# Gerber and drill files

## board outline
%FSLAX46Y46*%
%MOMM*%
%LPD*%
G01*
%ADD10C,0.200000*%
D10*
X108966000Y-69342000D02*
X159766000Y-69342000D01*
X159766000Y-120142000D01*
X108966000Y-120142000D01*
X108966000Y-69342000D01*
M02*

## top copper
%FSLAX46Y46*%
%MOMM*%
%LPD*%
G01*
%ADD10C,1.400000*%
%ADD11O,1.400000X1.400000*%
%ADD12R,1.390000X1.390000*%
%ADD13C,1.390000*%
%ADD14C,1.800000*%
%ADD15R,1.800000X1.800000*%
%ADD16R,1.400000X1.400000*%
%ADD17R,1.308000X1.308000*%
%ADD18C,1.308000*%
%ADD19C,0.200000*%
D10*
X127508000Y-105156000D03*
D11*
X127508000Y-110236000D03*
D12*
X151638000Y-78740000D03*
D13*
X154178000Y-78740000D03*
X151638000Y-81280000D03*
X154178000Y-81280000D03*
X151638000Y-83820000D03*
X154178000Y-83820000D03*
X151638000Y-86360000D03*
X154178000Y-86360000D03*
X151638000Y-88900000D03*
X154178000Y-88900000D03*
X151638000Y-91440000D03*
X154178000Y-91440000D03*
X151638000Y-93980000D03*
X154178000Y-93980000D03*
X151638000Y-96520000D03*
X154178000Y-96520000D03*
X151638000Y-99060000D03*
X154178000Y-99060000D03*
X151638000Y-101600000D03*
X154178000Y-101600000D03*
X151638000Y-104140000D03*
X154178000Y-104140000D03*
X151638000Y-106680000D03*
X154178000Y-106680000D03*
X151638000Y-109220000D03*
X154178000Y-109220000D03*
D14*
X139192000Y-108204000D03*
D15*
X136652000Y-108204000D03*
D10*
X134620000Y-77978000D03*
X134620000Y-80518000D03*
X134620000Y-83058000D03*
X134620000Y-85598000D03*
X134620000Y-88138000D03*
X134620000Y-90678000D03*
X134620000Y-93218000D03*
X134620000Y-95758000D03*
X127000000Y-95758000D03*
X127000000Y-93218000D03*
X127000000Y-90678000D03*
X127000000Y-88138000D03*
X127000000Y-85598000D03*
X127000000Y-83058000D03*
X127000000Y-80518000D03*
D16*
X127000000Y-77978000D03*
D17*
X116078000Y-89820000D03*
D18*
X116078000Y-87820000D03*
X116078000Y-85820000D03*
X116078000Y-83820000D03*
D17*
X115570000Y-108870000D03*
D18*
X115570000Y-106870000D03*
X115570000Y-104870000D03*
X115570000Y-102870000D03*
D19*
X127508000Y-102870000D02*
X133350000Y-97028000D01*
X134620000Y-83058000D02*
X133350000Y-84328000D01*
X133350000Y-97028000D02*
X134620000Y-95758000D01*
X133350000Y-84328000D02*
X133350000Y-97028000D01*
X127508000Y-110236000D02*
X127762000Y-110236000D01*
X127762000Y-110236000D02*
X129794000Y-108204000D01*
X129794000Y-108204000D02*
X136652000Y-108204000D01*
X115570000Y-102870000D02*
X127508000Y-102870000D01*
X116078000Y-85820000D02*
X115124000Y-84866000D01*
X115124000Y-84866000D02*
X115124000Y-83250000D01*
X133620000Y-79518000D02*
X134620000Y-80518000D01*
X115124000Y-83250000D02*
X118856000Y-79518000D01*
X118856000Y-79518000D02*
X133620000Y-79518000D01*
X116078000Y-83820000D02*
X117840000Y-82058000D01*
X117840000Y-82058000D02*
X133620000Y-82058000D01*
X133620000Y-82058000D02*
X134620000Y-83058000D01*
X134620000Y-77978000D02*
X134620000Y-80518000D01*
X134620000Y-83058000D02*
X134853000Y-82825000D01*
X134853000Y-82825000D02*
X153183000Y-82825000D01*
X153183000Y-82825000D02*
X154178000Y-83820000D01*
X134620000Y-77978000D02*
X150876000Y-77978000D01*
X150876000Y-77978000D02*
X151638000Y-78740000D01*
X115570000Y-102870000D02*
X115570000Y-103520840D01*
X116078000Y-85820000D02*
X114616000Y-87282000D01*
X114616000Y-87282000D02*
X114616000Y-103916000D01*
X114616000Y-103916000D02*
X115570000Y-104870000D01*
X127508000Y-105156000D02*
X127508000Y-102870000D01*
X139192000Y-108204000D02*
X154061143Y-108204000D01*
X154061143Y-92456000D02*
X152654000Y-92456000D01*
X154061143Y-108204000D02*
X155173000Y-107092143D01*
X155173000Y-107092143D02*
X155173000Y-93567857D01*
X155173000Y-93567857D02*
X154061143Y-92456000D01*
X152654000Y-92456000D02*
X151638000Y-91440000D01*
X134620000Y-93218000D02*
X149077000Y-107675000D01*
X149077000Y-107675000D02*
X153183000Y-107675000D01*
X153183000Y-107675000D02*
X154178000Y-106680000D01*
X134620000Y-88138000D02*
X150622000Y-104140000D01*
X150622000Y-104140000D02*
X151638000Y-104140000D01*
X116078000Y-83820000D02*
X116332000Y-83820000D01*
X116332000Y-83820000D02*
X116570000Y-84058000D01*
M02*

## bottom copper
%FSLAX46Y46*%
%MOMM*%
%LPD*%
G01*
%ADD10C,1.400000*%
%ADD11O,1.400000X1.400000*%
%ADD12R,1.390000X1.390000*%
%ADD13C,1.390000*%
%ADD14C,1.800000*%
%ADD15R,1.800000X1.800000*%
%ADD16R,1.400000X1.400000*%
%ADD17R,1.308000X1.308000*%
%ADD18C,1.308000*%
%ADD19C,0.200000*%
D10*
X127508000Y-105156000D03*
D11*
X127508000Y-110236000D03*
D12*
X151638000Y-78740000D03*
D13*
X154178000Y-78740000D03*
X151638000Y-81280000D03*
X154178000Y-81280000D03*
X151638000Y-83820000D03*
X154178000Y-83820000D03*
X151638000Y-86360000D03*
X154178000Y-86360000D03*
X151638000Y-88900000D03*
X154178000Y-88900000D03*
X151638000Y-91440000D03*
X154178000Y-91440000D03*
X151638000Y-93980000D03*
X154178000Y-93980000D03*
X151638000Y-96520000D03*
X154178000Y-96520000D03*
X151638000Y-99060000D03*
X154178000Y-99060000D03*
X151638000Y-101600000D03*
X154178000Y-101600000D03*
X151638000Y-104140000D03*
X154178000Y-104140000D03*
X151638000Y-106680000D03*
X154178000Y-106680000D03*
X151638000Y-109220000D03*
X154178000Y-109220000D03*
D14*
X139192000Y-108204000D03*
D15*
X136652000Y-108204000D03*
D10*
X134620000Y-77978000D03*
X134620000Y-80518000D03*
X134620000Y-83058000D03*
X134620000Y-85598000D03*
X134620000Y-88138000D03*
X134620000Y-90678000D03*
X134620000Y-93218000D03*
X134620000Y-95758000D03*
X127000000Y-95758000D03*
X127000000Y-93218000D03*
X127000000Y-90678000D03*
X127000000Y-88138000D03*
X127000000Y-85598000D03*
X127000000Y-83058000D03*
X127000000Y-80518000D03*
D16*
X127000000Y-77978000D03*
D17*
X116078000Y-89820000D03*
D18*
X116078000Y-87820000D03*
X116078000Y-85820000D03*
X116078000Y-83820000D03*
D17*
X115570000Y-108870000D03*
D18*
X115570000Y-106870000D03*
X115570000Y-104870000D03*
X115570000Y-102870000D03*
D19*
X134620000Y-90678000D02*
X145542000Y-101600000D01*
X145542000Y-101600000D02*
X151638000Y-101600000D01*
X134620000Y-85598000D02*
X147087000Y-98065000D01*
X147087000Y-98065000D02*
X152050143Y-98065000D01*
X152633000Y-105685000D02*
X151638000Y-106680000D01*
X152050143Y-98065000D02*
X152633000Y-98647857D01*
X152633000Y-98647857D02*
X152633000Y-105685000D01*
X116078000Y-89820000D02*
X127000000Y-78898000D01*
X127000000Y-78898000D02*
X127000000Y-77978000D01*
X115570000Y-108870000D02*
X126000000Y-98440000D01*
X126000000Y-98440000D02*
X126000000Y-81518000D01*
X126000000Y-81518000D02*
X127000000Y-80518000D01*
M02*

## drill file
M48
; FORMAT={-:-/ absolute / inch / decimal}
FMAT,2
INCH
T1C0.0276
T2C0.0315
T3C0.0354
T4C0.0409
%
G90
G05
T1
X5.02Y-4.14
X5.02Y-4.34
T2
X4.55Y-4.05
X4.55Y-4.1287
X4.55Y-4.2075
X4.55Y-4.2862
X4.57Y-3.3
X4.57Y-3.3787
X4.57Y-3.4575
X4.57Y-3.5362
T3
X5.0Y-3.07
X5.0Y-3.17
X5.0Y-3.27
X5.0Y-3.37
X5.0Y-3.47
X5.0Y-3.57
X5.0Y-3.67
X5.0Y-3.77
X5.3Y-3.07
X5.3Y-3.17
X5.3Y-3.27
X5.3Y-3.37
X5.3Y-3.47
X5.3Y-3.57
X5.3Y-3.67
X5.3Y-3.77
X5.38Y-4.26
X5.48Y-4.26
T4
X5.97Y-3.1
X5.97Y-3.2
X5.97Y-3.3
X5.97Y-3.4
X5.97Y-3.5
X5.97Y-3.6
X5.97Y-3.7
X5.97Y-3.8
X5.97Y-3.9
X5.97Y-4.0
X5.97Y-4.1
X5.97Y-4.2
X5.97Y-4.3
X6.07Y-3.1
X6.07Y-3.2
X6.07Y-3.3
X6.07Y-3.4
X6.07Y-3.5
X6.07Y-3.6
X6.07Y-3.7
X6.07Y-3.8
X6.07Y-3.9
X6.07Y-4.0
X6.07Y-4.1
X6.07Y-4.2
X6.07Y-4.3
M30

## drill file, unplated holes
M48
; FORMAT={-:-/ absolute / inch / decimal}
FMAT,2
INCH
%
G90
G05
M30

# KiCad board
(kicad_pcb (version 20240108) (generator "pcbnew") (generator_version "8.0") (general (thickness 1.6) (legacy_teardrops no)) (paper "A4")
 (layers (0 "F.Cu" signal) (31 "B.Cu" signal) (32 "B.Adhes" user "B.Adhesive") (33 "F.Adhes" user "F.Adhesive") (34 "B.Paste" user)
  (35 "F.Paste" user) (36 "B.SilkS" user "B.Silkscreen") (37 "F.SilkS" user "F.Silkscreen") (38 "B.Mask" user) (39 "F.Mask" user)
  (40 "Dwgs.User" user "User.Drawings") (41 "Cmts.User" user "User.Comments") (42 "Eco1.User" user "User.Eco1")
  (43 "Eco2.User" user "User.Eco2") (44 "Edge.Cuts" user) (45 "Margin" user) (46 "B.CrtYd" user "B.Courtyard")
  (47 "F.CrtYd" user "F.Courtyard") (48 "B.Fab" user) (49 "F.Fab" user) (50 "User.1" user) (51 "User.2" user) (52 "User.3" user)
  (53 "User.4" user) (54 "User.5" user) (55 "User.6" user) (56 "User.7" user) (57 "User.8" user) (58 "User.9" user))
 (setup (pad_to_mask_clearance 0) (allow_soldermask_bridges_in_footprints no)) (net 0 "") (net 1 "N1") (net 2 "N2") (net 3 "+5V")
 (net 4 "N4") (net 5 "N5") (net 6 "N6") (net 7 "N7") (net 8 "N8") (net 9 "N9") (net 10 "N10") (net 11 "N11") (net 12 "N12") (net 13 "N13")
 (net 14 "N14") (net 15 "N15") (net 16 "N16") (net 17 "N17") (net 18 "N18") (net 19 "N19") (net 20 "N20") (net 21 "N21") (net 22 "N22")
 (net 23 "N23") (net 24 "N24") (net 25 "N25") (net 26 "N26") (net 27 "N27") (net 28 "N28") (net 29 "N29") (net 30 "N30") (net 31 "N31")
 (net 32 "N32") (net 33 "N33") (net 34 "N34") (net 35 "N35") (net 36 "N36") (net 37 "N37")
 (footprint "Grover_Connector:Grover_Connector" (layer "F.Cu") (at 115.57 105.87 90)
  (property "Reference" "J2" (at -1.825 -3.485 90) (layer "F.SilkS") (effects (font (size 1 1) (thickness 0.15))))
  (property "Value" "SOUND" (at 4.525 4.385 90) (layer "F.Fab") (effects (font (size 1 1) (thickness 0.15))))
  (pad "1" thru_hole rect (at -3 0 90) (size 1.308 1.308) (drill 0.8) (layers "*.Cu" "*.Mask") (remove_unused_layers no) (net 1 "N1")
   (solder_mask_margin 0.102))
  (pad "2" thru_hole circle (at -1 0 90) (size 1.308 1.308) (drill 0.8) (layers "*.Cu" "*.Mask") (remove_unused_layers no) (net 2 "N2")
   (solder_mask_margin 0.102))
  (pad "3" thru_hole circle (at 1 0 90) (size 1.308 1.308) (drill 0.8) (layers "*.Cu" "*.Mask") (remove_unused_layers no) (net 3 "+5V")
   (solder_mask_margin 0.102))
  (pad "4" thru_hole circle (at 3 0 90) (size 1.308 1.308) (drill 0.8) (layers "*.Cu" "*.Mask") (remove_unused_layers no) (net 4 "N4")
   (solder_mask_margin 0.102)))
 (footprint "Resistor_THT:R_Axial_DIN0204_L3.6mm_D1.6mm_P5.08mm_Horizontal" (layer "F.Cu") (at 127.508 105.156 -90)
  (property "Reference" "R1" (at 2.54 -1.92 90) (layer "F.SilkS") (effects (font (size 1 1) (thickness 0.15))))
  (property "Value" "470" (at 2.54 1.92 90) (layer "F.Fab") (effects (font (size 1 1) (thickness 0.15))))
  (pad "1" thru_hole circle (at 0 0 270) (size 1.4 1.4) (drill 0.7) (layers "*.Cu" "*.Mask") (remove_unused_layers no) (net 4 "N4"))
  (pad "2" thru_hole oval (at 5.08 0 270) (size 1.4 1.4) (drill 0.7) (layers "*.Cu" "*.Mask") (remove_unused_layers no) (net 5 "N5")))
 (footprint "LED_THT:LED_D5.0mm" (layer "F.Cu") (at 136.652 108.204)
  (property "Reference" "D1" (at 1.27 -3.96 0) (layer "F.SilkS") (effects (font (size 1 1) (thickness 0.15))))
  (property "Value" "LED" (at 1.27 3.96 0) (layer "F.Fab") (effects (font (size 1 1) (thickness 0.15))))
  (pad "1" thru_hole rect (at 0 0) (size 1.8 1.8) (drill 0.9) (layers "*.Cu" "*.Mask") (remove_unused_layers no) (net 5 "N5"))
  (pad "2" thru_hole circle (at 2.54 0) (size 1.8 1.8) (drill 0.9) (layers "*.Cu" "*.Mask") (remove_unused_layers no) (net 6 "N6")))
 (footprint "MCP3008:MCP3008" (layer "F.Cu") (at 130.81 86.868 -90)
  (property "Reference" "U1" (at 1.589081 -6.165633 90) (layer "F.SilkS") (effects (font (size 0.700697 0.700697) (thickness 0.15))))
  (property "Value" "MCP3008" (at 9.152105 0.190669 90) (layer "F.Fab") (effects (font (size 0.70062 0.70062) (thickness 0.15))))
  (pad "1" thru_hole rect (at -8.89 3.81 270) (size 1.4 1.4) (drill 0.9) (layers "*.Cu" "*.Mask") (remove_unused_layers no) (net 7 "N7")
   (solder_mask_margin 0.102))
  (pad "2" thru_hole circle (at -6.35 3.81 270) (size 1.4 1.4) (drill 0.9) (layers "*.Cu" "*.Mask") (remove_unused_layers no) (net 1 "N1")
   (solder_mask_margin 0.102))
  (pad "3" thru_hole circle (at -3.81 3.81 270) (size 1.4 1.4) (drill 0.9) (layers "*.Cu" "*.Mask") (remove_unused_layers no) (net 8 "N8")
   (solder_mask_margin 0.102))
  (pad "4" thru_hole circle (at -1.27 3.81 270) (size 1.4 1.4) (drill 0.9) (layers "*.Cu" "*.Mask") (remove_unused_layers no) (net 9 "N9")
   (solder_mask_margin 0.102))
  (pad "5" thru_hole circle (at 1.27 3.81 270) (size 1.4 1.4) (drill 0.9) (layers "*.Cu" "*.Mask") (remove_unused_layers no) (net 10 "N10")
   (solder_mask_margin 0.102))
  (pad "6" thru_hole circle (at 3.81 3.81 270) (size 1.4 1.4) (drill 0.9) (layers "*.Cu" "*.Mask") (remove_unused_layers no) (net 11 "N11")
   (solder_mask_margin 0.102))
  (pad "7" thru_hole circle (at 6.35 3.81 270) (size 1.4 1.4) (drill 0.9) (layers "*.Cu" "*.Mask") (remove_unused_layers no) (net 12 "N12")
   (solder_mask_margin 0.102))
  (pad "8" thru_hole circle (at 8.89 3.81 270) (size 1.4 1.4) (drill 0.9) (layers "*.Cu" "*.Mask") (remove_unused_layers no) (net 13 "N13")
   (solder_mask_margin 0.102))
  (pad "9" thru_hole circle (at 8.89 -3.81 270) (size 1.4 1.4) (drill 0.9) (layers "*.Cu" "*.Mask") (remove_unused_layers no) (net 4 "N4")
   (solder_mask_margin 0.102))
  (pad "10" thru_hole circle (at 6.35 -3.81 270) (size 1.4 1.4) (drill 0.9) (layers "*.Cu" "*.Mask") (remove_unused_layers no)
   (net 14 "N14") (solder_mask_margin 0.102))
  (pad "11" thru_hole circle (at 3.81 -3.81 270) (size 1.4 1.4) (drill 0.9) (layers "*.Cu" "*.Mask") (remove_unused_layers no)
   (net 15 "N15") (solder_mask_margin 0.102))
  (pad "12" thru_hole circle (at 1.27 -3.81 270) (size 1.4 1.4) (drill 0.9) (layers "*.Cu" "*.Mask") (remove_unused_layers no)
   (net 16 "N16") (solder_mask_margin 0.102))
  (pad "13" thru_hole circle (at -1.27 -3.81 270) (size 1.4 1.4) (drill 0.9) (layers "*.Cu" "*.Mask") (remove_unused_layers no)
   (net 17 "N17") (solder_mask_margin 0.102))
  (pad "14" thru_hole circle (at -3.81 -3.81 270) (size 1.4 1.4) (drill 0.9) (layers "*.Cu" "*.Mask") (remove_unused_layers no) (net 4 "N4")
   (solder_mask_margin 0.102))
  (pad "15" thru_hole circle (at -6.35 -3.81 270) (size 1.4 1.4) (drill 0.9) (layers "*.Cu" "*.Mask") (remove_unused_layers no)
   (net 3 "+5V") (solder_mask_margin 0.102))
  (pad "16" thru_hole circle (at -8.89 -3.81 270) (size 1.4 1.4) (drill 0.9) (layers "*.Cu" "*.Mask") (remove_unused_layers no)
   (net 3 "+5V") (solder_mask_margin 0.102)))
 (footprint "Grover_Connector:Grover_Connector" (layer "F.Cu") (at 116.078 86.82 90)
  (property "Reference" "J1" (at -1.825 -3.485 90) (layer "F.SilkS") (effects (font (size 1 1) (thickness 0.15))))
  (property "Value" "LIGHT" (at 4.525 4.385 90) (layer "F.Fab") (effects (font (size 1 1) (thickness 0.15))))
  (pad "1" thru_hole rect (at -3 0 90) (size 1.308 1.308) (drill 0.8) (layers "*.Cu" "*.Mask") (remove_unused_layers no) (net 7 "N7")
   (solder_mask_margin 0.102))
  (pad "2" thru_hole circle (at -1 0 90) (size 1.308 1.308) (drill 0.8) (layers "*.Cu" "*.Mask") (remove_unused_layers no) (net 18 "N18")
   (solder_mask_margin 0.102))
  (pad "3" thru_hole circle (at 1 0 90) (size 1.308 1.308) (drill 0.8) (layers "*.Cu" "*.Mask") (remove_unused_layers no) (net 3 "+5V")
   (solder_mask_margin 0.102))
  (pad "4" thru_hole circle (at 3 0 90) (size 1.308 1.308) (drill 0.8) (layers "*.Cu" "*.Mask") (remove_unused_layers no) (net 4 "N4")
   (solder_mask_margin 0.102)))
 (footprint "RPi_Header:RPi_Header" (layer "B.Cu") (at 151.638 78.74 90)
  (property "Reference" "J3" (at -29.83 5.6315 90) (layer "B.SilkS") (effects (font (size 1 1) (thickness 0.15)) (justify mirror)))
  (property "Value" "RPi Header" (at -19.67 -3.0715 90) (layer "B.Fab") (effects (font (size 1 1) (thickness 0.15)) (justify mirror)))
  (pad "01" thru_hole rect (at 0 0 90) (size 1.39 1.39) (drill 1.04) (layers "*.Cu" "*.Mask") (remove_unused_layers no) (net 3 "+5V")
   (solder_mask_margin 0.102))
  (pad "02" thru_hole circle (at 0 2.54 90) (size 1.39 1.39) (drill 1.04) (layers "*.Cu" "*.Mask") (remove_unused_layers no) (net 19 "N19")
   (solder_mask_margin 0.102))
  (pad "03" thru_hole circle (at -2.54 0 90) (size 1.39 1.39) (drill 1.04) (layers "*.Cu" "*.Mask") (remove_unused_layers no) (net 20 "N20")
   (solder_mask_margin 0.102))
  (pad "04" thru_hole circle (at -2.54 2.54 90) (size 1.39 1.39) (drill 1.04) (layers "*.Cu" "*.Mask") (remove_unused_layers no)
   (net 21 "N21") (solder_mask_margin 0.102))
  (pad "05" thru_hole circle (at -5.08 0 90) (size 1.39 1.39) (drill 1.04) (layers "*.Cu" "*.Mask") (remove_unused_layers no) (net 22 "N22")
   (solder_mask_margin 0.102))
  (pad "06" thru_hole circle (at -5.08 2.54 90) (size 1.39 1.39) (drill 1.04) (layers "*.Cu" "*.Mask") (remove_unused_layers no)
   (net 4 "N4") (solder_mask_margin 0.102))
  (pad "07" thru_hole circle (at -7.62 0 90) (size 1.39 1.39) (drill 1.04) (layers "*.Cu" "*.Mask") (remove_unused_layers no) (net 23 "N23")
   (solder_mask_margin 0.102))
  (pad "08" thru_hole circle (at -7.62 2.54 90) (size 1.39 1.39) (drill 1.04) (layers "*.Cu" "*.Mask") (remove_unused_layers no)
   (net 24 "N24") (solder_mask_margin 0.102))
  (pad "09" thru_hole circle (at -10.16 0 90) (size 1.39 1.39) (drill 1.04) (layers "*.Cu" "*.Mask") (remove_unused_layers no)
   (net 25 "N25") (solder_mask_margin 0.102))
  (pad "10" thru_hole circle (at -10.16 2.54 90) (size 1.39 1.39) (drill 1.04) (layers "*.Cu" "*.Mask") (remove_unused_layers no)
   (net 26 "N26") (solder_mask_margin 0.102))
  (pad "11" thru_hole circle (at -12.7 0 90) (size 1.39 1.39) (drill 1.04) (layers "*.Cu" "*.Mask") (remove_unused_layers no) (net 6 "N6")
   (solder_mask_margin 0.102))
  (pad "12" thru_hole circle (at -12.7 2.54 90) (size 1.39 1.39) (drill 1.04) (layers "*.Cu" "*.Mask") (remove_unused_layers no)
   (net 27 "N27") (solder_mask_margin 0.102))
  (pad "13" thru_hole circle (at -15.24 0 90) (size 1.39 1.39) (drill 1.04) (layers "*.Cu" "*.Mask") (remove_unused_layers no)
   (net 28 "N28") (solder_mask_margin 0.102))
  (pad "14" thru_hole circle (at -15.24 2.54 90) (size 1.39 1.39) (drill 1.04) (layers "*.Cu" "*.Mask") (remove_unused_layers no)
   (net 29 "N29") (solder_mask_margin 0.102))
  (pad "15" thru_hole circle (at -17.78 0 90) (size 1.39 1.39) (drill 1.04) (layers "*.Cu" "*.Mask") (remove_unused_layers no)
   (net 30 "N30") (solder_mask_margin 0.102))
  (pad "16" thru_hole circle (at -17.78 2.54 90) (size 1.39 1.39) (drill 1.04) (layers "*.Cu" "*.Mask") (remove_unused_layers no)
   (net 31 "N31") (solder_mask_margin 0.102))
  (pad "17" thru_hole circle (at -20.32 0 90) (size 1.39 1.39) (drill 1.04) (layers "*.Cu" "*.Mask") (remove_unused_layers no)
   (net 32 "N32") (solder_mask_margin 0.102))
  (pad "18" thru_hole circle (at -20.32 2.54 90) (size 1.39 1.39) (drill 1.04) (layers "*.Cu" "*.Mask") (remove_unused_layers no)
   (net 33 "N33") (solder_mask_margin 0.102))
  (pad "19" thru_hole circle (at -22.86 0 90) (size 1.39 1.39) (drill 1.04) (layers "*.Cu" "*.Mask") (remove_unused_layers no)
   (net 15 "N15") (solder_mask_margin 0.102))
  (pad "20" thru_hole circle (at -22.86 2.54 90) (size 1.39 1.39) (drill 1.04) (layers "*.Cu" "*.Mask") (remove_unused_layers no)
   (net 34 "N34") (solder_mask_margin 0.102))
  (pad "21" thru_hole circle (at -25.4 0 90) (size 1.39 1.39) (drill 1.04) (layers "*.Cu" "*.Mask") (remove_unused_layers no) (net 16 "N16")
   (solder_mask_margin 0.102))
  (pad "22" thru_hole circle (at -25.4 2.54 90) (size 1.39 1.39) (drill 1.04) (layers "*.Cu" "*.Mask") (remove_unused_layers no)
   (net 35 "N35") (solder_mask_margin 0.102))
  (pad "23" thru_hole circle (at -27.94 0 90) (size 1.39 1.39) (drill 1.04) (layers "*.Cu" "*.Mask") (remove_unused_layers no)
   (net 17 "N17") (solder_mask_margin 0.102))
  (pad "24" thru_hole circle (at -27.94 2.54 90) (size 1.39 1.39) (drill 1.04) (layers "*.Cu" "*.Mask") (remove_unused_layers no)
   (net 14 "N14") (solder_mask_margin 0.102))
  (pad "25" thru_hole circle (at -30.48 0 90) (size 1.39 1.39) (drill 1.04) (layers "*.Cu" "*.Mask") (remove_unused_layers no)
   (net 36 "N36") (solder_mask_margin 0.102))
  (pad "26" thru_hole circle (at -30.48 2.54 90) (size 1.39 1.39) (drill 1.04) (layers "*.Cu" "*.Mask") (remove_unused_layers no)
   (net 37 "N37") (solder_mask_margin 0.102)))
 (gr_rect (start 108.966 69.342) (end 159.766 120.142) (stroke (width 0.2) (type default)) (fill none) (layer "Edge.Cuts"))
 (segment (start 129.794 108.204) (end 136.652 108.204) (width 0.2) (layer "F.Cu") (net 5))
 (segment (start 127.762 110.236) (end 129.794 108.204) (width 0.2) (layer "F.Cu") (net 5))
 (segment (start 127.508 110.236) (end 127.762 110.236) (width 0.2) (layer "F.Cu") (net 5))
 (segment (start 139.192 108.204) (end 154.061143 108.204) (width 0.2) (layer "F.Cu") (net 6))
 (segment (start 155.173 107.092143) (end 155.173 93.567857) (width 0.2) (layer "F.Cu") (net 6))
 (segment (start 154.061143 108.204) (end 155.173 107.092143) (width 0.2) (layer "F.Cu") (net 6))
 (segment (start 154.061143 92.456) (end 152.654 92.456) (width 0.2) (layer "F.Cu") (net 6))
 (segment (start 155.173 93.567857) (end 154.061143 92.456) (width 0.2) (layer "F.Cu") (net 6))
 (segment (start 152.654 92.456) (end 151.638 91.44) (width 0.2) (layer "F.Cu") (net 6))
 (segment (start 116.078 83.82) (end 116.332 83.82) (width 0.2) (layer "F.Cu") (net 4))
 (segment (start 153.183 82.825) (end 154.178 83.82) (width 0.2) (layer "F.Cu") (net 4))
 (segment (start 127.508 105.156) (end 127.508 102.87) (width 0.2) (layer "F.Cu") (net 4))
 (segment (start 133.62 82.058) (end 134.62 83.058) (width 0.2) (layer "F.Cu") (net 4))
 (segment (start 133.35 97.028) (end 134.62 95.758) (width 0.2) (layer "F.Cu") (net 4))
 (segment (start 115.57 102.87) (end 127.508 102.87) (width 0.2) (layer "F.Cu") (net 4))
 (segment (start 116.332 83.82) (end 116.57 84.058) (width 0.2) (layer "F.Cu") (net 4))
 (segment (start 134.62 83.058) (end 134.853 82.825) (width 0.2) (layer "F.Cu") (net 4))
 (segment (start 117.84 82.058) (end 133.62 82.058) (width 0.2) (layer "F.Cu") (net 4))
 (segment (start 133.35 84.328) (end 133.35 97.028) (width 0.2) (layer "F.Cu") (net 4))
 (segment (start 116.078 83.82) (end 117.84 82.058) (width 0.2) (layer "F.Cu") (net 4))
 (segment (start 115.57 102.87) (end 115.57 103.52084) (width 0.2) (layer "F.Cu") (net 4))
 (segment (start 134.853 82.825) (end 153.183 82.825) (width 0.2) (layer "F.Cu") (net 4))
 (segment (start 127.508 102.87) (end 133.35 97.028) (width 0.2) (layer "F.Cu") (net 4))
 (segment (start 134.62 83.058) (end 133.35 84.328) (width 0.2) (layer "F.Cu") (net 4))
 (segment (start 127 78.898) (end 127 77.978) (width 0.2) (layer "B.Cu") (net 7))
 (segment (start 116.078 89.82) (end 127 78.898) (width 0.2) (layer "B.Cu") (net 7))
 (segment (start 134.62 77.978) (end 150.876 77.978) (width 0.2) (layer "F.Cu") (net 3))
 (segment (start 114.616 87.282) (end 114.616 103.916) (width 0.2) (layer "F.Cu") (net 3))
 (segment (start 133.62 79.518) (end 134.62 80.518) (width 0.2) (layer "F.Cu") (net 3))
 (segment (start 116.078 85.82) (end 114.616 87.282) (width 0.2) (layer "F.Cu") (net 3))
 (segment (start 118.856 79.518) (end 133.62 79.518) (width 0.2) (layer "F.Cu") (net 3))
 (segment (start 115.124 84.866) (end 115.124 83.25) (width 0.2) (layer "F.Cu") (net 3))
 (segment (start 150.876 77.978) (end 151.638 78.74) (width 0.2) (layer "F.Cu") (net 3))
 (segment (start 134.62 77.978) (end 134.62 80.518) (width 0.2) (layer "F.Cu") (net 3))
 (segment (start 115.124 83.25) (end 118.856 79.518) (width 0.2) (layer "F.Cu") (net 3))
 (segment (start 116.078 85.82) (end 115.124 84.866) (width 0.2) (layer "F.Cu") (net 3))
 (segment (start 114.616 103.916) (end 115.57 104.87) (width 0.2) (layer "F.Cu") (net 3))
 (segment (start 126 81.518) (end 127 80.518) (width 0.2) (layer "B.Cu") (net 1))
 (segment (start 126 98.44) (end 126 81.518) (width 0.2) (layer "B.Cu") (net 1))
 (segment (start 115.57 108.87) (end 126 98.44) (width 0.2) (layer "B.Cu") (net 1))
 (segment (start 147.087 98.065) (end 152.050143 98.065) (width 0.2) (layer "B.Cu") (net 17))
 (segment (start 152.633 98.647857) (end 152.633 105.685) (width 0.2) (layer "B.Cu") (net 17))
 (segment (start 134.62 85.598) (end 147.087 98.065) (width 0.2) (layer "B.Cu") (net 17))
 (segment (start 152.633 105.685) (end 151.638 106.68) (width 0.2) (layer "B.Cu") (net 17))
 (segment (start 152.050143 98.065) (end 152.633 98.647857) (width 0.2) (layer "B.Cu") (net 17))
 (segment (start 150.622 104.14) (end 151.638 104.14) (width 0.2) (layer "F.Cu") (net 16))
 (segment (start 134.62 88.138) (end 150.622 104.14) (width 0.2) (layer "F.Cu") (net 16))
 (segment (start 134.62 90.678) (end 145.542 101.6) (width 0.2) (layer "B.Cu") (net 15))
 (segment (start 145.542 101.6) (end 151.638 101.6) (width 0.2) (layer "B.Cu") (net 15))
 (segment (start 153.183 107.675) (end 154.178 106.68) (width 0.2) (layer "F.Cu") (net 14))
 (segment (start 134.62 93.218) (end 149.077 107.675) (width 0.2) (layer "F.Cu") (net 14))
 (segment (start 149.077 107.675) (end 153.183 107.675) (width 0.2) (layer "F.Cu") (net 14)))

